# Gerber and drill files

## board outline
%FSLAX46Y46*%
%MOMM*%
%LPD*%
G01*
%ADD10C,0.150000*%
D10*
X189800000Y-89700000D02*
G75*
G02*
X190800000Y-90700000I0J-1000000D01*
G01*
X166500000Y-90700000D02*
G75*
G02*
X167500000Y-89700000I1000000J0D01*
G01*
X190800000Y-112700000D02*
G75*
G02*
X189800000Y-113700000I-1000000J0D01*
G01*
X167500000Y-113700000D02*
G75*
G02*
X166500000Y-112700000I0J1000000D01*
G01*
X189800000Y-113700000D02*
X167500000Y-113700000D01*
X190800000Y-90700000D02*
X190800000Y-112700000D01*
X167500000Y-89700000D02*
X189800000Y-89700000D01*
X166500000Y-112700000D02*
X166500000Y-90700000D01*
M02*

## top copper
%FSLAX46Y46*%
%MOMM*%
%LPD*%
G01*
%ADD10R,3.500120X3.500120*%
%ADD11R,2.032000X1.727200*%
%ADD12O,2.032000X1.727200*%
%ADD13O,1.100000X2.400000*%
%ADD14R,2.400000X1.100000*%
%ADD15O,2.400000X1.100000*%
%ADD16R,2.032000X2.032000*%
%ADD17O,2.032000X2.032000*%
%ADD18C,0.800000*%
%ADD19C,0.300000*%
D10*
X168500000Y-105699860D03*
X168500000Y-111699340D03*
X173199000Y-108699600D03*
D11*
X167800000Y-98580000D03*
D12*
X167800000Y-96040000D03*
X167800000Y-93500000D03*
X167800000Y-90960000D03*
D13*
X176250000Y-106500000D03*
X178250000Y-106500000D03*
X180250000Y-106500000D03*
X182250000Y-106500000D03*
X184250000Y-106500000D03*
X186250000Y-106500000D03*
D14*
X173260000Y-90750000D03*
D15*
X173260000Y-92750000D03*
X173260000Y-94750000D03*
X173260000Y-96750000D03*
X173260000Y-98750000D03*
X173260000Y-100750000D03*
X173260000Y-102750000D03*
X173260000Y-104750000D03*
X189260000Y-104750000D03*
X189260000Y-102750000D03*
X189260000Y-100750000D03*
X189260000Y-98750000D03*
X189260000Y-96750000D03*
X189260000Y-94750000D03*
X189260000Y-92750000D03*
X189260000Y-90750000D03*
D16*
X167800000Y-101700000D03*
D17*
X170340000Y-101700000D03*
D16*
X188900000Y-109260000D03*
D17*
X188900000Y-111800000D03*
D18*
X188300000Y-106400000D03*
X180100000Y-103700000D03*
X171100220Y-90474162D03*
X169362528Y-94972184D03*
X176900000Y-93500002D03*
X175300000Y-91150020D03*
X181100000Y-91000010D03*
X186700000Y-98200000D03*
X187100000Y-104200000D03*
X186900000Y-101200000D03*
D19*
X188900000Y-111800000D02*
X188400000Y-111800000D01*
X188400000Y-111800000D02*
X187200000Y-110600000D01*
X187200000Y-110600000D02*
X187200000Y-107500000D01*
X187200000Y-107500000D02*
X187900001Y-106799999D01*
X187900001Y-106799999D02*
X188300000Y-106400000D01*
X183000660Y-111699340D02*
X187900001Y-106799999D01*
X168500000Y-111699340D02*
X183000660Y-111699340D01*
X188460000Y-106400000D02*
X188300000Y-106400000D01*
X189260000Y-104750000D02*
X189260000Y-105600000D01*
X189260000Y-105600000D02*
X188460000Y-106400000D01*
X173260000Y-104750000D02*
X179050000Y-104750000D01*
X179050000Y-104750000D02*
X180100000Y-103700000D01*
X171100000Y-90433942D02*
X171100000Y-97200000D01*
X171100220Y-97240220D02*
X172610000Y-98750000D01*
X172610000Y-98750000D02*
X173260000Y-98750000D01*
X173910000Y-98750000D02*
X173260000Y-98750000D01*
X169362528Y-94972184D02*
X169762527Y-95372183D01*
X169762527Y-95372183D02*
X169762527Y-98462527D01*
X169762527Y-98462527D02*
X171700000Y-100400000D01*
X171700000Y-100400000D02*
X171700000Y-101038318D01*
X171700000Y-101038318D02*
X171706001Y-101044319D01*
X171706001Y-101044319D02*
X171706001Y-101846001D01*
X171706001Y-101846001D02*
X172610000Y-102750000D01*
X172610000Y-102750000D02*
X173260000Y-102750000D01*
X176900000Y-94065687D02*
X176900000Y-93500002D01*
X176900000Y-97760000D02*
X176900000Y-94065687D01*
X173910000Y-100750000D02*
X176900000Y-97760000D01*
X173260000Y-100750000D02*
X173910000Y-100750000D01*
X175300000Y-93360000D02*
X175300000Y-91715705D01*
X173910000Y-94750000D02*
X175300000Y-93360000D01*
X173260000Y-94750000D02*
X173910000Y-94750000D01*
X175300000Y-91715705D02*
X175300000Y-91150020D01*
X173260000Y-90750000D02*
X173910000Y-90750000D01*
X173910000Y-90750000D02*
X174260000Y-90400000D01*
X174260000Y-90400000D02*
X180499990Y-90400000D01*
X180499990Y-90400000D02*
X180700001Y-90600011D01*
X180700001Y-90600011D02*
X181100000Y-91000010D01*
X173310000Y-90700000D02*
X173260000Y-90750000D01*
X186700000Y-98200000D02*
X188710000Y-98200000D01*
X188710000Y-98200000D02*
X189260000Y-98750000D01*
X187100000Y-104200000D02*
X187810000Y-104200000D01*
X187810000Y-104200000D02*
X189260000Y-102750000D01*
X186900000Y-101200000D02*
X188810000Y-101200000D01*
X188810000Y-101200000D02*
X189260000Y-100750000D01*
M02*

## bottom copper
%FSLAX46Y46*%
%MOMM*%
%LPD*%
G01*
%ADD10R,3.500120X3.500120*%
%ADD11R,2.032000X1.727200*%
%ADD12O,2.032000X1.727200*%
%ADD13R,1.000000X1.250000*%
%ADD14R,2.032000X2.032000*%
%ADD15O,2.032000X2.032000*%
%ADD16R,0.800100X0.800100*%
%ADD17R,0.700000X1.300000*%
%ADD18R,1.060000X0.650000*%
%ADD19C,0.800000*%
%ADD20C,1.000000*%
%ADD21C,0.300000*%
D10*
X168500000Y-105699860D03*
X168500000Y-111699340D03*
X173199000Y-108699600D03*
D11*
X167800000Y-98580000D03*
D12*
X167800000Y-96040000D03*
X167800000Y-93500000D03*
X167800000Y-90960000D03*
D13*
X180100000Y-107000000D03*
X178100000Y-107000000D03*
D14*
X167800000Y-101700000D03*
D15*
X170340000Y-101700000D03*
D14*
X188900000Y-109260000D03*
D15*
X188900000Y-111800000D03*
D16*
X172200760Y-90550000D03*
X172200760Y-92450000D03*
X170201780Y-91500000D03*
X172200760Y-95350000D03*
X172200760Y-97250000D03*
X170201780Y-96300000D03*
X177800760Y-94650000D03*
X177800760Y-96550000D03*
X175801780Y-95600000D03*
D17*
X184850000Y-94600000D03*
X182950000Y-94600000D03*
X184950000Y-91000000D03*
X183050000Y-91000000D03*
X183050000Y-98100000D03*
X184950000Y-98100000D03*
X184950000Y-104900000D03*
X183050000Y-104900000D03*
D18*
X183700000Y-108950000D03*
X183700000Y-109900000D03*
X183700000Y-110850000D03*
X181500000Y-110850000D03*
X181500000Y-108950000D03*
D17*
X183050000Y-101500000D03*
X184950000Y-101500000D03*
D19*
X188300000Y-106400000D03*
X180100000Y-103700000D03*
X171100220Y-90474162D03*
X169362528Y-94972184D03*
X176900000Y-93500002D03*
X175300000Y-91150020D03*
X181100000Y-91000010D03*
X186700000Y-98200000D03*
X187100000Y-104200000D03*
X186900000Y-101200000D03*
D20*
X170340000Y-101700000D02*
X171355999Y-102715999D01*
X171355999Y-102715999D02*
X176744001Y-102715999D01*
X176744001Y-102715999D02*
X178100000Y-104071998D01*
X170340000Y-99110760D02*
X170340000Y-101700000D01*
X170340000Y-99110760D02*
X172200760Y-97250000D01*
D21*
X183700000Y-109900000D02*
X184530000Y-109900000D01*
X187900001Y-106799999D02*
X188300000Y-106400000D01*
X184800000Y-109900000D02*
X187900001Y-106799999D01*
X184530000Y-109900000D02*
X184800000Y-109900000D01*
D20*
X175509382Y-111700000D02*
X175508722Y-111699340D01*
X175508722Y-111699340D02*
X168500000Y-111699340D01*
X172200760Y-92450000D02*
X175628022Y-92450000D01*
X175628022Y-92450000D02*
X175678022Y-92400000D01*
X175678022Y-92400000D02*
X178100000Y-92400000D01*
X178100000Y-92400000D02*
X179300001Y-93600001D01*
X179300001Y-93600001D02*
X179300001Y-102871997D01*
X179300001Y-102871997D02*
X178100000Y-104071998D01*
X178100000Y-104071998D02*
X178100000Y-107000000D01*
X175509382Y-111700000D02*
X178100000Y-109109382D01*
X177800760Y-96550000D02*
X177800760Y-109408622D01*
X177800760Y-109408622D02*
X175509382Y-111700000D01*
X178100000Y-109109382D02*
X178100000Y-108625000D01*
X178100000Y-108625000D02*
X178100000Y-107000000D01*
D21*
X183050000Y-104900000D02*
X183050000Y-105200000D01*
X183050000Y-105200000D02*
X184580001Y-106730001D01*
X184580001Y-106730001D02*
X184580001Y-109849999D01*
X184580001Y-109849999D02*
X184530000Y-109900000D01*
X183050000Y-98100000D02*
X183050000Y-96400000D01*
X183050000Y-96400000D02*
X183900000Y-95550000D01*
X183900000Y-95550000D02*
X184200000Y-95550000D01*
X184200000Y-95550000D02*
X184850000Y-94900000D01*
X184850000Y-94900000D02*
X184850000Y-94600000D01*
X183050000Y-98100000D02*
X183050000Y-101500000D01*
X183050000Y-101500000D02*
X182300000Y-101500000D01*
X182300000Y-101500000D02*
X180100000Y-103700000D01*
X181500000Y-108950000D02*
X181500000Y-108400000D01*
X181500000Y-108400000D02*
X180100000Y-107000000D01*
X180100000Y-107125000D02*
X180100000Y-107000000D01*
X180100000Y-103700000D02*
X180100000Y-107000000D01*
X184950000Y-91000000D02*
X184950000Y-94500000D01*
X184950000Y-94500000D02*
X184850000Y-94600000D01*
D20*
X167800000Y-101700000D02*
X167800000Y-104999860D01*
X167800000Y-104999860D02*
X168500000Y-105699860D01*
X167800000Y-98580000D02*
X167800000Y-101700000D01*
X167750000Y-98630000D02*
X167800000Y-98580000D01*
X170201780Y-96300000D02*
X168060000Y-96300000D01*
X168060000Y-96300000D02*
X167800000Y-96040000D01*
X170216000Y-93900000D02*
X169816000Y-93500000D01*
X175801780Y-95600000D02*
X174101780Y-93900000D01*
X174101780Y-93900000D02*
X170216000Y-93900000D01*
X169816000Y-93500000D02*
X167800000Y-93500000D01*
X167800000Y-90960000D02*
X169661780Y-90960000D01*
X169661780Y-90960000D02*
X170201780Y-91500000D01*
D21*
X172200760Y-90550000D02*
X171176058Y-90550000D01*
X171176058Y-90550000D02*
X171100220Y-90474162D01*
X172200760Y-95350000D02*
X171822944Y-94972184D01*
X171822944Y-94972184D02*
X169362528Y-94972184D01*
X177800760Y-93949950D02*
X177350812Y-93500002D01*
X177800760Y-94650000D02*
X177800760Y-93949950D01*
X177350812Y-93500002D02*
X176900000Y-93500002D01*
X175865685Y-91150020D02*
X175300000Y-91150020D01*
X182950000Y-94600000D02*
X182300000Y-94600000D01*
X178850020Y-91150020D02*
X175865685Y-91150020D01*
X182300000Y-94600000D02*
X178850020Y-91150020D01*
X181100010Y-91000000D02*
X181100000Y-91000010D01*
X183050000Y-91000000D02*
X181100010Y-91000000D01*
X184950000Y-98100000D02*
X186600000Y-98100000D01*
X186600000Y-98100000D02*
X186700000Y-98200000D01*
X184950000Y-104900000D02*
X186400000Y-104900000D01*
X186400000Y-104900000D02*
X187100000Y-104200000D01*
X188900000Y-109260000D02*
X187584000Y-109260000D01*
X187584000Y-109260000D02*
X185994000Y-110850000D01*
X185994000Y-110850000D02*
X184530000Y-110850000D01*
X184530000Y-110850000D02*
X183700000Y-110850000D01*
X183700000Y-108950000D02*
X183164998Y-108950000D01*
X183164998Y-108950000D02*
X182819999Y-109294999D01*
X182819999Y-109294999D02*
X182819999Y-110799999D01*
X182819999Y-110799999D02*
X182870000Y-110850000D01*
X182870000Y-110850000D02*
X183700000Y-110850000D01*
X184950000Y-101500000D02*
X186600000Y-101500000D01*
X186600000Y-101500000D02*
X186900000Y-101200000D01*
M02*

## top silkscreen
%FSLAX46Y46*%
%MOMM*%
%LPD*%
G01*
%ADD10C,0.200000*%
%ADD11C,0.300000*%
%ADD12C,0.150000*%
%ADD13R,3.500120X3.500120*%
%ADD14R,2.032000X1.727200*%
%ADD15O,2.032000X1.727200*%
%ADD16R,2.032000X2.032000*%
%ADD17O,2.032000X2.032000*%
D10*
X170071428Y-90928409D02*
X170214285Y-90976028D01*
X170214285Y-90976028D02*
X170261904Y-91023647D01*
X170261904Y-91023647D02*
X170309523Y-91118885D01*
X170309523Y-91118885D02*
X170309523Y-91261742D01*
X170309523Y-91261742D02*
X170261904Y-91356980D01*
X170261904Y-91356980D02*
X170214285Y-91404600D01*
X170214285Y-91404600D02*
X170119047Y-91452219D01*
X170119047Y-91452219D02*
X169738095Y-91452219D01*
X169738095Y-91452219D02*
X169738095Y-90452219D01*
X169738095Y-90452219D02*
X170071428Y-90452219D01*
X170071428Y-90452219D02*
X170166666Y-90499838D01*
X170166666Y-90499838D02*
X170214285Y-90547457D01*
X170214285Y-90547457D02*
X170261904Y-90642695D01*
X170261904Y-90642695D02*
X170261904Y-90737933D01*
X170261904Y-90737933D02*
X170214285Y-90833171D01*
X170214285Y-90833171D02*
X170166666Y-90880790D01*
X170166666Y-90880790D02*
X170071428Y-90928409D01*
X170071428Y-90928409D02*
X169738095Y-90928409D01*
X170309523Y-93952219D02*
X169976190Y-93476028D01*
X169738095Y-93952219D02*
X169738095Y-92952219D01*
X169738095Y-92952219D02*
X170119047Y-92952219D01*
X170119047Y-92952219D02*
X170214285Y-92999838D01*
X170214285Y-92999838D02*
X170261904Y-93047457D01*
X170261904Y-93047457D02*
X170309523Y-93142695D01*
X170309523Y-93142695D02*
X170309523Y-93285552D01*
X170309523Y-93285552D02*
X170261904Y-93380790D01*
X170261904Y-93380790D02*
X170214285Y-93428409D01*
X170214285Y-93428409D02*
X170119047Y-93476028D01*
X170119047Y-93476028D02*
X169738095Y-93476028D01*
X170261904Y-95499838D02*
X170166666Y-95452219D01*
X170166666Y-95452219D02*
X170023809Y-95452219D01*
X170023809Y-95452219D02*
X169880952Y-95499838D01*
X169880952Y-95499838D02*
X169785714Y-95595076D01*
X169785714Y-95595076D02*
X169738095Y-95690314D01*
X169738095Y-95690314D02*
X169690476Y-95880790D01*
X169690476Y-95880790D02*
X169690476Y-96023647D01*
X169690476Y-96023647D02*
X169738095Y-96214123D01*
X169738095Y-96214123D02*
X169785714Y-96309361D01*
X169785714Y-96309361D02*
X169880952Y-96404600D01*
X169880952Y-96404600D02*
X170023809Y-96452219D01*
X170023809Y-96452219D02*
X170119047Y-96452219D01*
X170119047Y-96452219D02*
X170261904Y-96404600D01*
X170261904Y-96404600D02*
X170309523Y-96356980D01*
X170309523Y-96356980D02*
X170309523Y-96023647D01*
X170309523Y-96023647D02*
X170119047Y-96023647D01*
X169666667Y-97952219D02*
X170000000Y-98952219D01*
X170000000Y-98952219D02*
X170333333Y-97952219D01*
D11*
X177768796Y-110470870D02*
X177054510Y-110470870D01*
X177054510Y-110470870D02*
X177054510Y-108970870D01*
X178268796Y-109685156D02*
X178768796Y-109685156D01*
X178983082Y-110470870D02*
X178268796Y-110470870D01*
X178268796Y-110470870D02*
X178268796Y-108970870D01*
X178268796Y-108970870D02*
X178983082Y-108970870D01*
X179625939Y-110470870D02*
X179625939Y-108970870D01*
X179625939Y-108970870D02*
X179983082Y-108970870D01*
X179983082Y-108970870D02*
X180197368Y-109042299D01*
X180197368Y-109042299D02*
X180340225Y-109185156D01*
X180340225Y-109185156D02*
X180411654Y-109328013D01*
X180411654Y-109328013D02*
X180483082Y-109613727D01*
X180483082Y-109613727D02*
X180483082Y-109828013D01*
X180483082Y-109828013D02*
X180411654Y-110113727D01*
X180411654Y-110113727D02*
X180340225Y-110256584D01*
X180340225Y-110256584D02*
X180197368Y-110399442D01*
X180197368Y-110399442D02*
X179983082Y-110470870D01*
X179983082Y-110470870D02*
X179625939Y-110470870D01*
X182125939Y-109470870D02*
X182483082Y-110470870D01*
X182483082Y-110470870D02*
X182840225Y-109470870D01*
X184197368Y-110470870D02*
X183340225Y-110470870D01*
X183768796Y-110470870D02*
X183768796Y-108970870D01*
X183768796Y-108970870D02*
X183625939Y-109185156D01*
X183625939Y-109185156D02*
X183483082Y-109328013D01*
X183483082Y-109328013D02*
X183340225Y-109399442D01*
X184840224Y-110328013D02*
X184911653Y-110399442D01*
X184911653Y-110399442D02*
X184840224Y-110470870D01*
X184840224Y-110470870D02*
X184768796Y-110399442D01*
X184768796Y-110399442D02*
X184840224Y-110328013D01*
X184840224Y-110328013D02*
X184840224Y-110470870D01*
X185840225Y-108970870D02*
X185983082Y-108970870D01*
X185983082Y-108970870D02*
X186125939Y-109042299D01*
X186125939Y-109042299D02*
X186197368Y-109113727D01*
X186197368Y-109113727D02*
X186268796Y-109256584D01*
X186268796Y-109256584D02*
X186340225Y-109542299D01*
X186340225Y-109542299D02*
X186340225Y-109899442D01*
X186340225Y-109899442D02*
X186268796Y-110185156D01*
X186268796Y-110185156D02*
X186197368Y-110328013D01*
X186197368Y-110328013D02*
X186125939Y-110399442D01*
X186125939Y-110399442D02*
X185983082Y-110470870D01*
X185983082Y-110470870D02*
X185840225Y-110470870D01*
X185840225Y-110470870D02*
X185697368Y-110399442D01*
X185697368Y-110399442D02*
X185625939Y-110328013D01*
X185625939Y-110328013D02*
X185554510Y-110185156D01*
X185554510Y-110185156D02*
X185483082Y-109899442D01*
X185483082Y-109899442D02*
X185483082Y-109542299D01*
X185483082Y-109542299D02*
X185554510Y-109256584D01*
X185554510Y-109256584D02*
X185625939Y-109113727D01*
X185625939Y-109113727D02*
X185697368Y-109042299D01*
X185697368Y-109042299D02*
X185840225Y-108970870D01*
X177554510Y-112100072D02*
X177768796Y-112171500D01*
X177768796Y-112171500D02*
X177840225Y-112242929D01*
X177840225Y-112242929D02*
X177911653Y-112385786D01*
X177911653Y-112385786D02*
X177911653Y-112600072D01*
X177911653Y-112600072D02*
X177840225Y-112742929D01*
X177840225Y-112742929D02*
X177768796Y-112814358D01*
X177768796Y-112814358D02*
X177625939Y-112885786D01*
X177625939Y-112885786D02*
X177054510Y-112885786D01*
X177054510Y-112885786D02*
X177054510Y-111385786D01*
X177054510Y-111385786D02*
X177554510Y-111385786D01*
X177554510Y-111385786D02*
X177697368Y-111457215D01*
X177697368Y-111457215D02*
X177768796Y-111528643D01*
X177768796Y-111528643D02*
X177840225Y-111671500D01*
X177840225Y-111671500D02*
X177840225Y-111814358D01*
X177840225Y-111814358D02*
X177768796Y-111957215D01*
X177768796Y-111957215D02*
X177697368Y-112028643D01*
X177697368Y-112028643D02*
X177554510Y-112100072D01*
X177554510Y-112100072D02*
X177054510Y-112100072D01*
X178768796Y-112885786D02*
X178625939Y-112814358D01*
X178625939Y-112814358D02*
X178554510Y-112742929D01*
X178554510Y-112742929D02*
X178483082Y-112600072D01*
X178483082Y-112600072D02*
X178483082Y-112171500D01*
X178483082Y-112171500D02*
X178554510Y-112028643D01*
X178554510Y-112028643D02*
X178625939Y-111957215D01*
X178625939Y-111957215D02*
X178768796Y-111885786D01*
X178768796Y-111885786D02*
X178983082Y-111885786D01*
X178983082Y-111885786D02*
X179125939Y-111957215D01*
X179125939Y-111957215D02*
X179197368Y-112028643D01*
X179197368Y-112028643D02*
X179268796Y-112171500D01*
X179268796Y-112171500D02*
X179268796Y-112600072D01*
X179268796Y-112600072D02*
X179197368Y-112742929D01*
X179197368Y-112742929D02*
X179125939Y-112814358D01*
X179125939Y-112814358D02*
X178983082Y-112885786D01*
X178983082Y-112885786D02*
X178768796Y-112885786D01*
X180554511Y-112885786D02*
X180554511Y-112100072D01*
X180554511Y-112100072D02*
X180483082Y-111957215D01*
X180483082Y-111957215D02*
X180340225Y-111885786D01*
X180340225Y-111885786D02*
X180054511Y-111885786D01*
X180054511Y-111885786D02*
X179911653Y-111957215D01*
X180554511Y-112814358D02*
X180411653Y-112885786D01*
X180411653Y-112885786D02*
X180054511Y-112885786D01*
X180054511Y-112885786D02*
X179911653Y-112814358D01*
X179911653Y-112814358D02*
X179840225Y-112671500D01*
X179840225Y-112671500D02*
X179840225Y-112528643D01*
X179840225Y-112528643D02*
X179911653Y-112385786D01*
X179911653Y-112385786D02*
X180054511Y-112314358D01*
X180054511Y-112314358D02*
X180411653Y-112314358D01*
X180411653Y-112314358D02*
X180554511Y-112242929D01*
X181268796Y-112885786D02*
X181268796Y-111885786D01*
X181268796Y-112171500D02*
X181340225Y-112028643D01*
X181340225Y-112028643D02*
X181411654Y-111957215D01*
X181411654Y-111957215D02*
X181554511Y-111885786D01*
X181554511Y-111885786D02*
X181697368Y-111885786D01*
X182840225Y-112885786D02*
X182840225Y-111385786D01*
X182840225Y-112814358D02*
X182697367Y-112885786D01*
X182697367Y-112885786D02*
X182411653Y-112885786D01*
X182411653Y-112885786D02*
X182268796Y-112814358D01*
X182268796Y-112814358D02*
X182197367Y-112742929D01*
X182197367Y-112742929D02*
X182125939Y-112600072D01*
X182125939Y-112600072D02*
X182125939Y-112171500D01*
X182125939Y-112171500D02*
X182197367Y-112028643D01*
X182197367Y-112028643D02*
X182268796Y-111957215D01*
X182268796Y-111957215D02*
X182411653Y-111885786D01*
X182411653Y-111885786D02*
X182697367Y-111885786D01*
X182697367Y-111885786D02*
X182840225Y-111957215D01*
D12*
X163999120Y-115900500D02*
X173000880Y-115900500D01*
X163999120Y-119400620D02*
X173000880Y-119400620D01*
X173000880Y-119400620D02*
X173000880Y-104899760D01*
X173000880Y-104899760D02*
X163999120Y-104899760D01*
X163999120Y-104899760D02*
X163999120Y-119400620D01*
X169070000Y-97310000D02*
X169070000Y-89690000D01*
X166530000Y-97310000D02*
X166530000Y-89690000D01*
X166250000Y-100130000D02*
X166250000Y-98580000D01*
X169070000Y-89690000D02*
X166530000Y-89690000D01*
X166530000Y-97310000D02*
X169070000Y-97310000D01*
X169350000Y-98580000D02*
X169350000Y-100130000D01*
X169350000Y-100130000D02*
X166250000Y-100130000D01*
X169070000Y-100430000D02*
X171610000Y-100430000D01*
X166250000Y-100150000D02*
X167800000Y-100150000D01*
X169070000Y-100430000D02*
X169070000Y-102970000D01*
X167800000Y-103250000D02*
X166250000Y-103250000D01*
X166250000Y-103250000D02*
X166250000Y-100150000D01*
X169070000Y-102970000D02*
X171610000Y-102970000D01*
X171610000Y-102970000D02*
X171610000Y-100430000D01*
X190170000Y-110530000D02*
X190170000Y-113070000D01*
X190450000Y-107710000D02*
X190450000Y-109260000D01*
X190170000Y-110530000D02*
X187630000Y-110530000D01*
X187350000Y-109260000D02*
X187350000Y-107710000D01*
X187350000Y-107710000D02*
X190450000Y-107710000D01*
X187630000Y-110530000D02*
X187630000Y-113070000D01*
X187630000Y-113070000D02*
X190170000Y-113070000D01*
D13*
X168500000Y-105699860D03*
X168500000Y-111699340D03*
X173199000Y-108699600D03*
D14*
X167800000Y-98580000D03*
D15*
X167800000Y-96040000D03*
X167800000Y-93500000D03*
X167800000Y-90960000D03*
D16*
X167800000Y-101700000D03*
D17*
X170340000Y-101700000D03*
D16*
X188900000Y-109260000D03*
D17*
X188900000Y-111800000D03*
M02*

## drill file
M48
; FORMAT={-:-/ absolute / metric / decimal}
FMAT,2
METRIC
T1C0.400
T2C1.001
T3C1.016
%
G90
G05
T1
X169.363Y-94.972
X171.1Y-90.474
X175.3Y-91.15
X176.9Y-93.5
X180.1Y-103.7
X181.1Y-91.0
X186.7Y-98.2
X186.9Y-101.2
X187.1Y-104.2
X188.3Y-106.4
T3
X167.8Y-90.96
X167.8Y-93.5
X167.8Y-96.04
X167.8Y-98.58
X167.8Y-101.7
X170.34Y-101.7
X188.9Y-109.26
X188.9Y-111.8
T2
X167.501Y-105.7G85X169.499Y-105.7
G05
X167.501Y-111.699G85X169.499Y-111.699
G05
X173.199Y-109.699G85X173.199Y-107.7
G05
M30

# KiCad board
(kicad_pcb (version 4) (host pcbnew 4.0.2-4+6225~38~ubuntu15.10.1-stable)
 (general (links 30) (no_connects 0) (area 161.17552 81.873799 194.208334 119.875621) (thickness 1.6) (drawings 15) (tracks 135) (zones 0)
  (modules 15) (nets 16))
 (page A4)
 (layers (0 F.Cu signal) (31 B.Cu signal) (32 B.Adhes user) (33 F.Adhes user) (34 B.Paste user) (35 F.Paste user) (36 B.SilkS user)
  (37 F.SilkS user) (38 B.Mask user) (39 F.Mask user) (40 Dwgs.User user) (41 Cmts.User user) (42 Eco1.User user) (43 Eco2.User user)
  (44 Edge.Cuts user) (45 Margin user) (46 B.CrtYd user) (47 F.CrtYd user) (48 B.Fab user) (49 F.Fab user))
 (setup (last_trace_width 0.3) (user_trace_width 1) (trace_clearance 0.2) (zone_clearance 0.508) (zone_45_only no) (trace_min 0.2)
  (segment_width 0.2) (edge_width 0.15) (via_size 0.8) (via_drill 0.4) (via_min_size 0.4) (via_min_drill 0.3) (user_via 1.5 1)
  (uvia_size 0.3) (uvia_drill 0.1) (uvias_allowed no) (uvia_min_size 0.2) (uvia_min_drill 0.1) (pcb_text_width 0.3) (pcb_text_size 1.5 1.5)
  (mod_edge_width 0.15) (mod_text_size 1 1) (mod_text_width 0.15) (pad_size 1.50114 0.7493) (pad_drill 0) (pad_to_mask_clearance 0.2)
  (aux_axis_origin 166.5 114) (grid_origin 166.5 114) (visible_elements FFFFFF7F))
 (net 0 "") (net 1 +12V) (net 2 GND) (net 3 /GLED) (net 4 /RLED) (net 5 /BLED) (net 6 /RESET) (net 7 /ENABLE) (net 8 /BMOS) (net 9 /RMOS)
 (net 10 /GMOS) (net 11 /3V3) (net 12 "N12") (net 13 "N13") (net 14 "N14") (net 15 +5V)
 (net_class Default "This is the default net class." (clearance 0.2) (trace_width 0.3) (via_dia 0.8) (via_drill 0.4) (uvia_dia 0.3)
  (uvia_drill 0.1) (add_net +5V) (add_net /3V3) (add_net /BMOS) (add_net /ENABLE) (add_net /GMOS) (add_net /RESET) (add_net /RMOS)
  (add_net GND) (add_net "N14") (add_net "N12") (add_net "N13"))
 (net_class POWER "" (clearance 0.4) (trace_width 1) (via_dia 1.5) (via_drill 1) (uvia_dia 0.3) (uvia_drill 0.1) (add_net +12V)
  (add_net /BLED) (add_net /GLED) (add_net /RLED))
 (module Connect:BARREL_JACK (layer F.Cu) (at 168.5 111.9 90)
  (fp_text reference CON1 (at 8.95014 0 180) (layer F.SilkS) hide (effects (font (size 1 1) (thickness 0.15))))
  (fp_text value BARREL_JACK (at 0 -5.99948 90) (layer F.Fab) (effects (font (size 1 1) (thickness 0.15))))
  (fp_line (start -4.0005 -4.50088) (end -4.0005 4.50088) (layer F.SilkS) (width 0.15))
  (fp_line (start -7.50062 -4.50088) (end -7.50062 4.50088) (layer F.SilkS) (width 0.15))
  (fp_line (start -7.50062 4.50088) (end 7.00024 4.50088) (layer F.SilkS) (width 0.15))
  (fp_line (start 7.00024 4.50088) (end 7.00024 -4.50088) (layer F.SilkS) (width 0.15))
  (fp_line (start 7.00024 -4.50088) (end -7.50062 -4.50088) (layer F.SilkS) (width 0.15))
  (pad 1 thru_hole rect (at 6.20014 0 90) (size 3.50012 3.50012) (drill oval 1.00076 2.99974) (layers *.Cu *.Mask F.SilkS) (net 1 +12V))
  (pad 2 thru_hole rect (at 0.20066 0 90) (size 3.50012 3.50012) (drill oval 1.00076 2.99974) (layers *.Cu *.Mask F.SilkS) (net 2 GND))
  (pad 3 thru_hole rect (at 3.2004 4.699 90) (size 3.50012 3.50012) (drill oval 2.99974 1.00076) (layers *.Cu *.Mask F.SilkS)))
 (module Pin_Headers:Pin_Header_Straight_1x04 (layer F.Cu) (at 167.8 98.58 180)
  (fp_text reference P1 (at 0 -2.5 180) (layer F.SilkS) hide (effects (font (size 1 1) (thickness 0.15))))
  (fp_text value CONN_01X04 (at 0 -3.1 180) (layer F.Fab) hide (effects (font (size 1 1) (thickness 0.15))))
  (fp_line (start -1.27 1.27) (end -1.27 8.89) (layer F.SilkS) (width 0.15))
  (fp_line (start 1.27 1.27) (end 1.27 8.89) (layer F.SilkS) (width 0.15))
  (fp_line (start 1.55 -1.55) (end 1.55 0) (layer F.SilkS) (width 0.15))
  (fp_line (start -1.27 8.89) (end 1.27 8.89) (layer F.SilkS) (width 0.15))
  (fp_line (start 1.27 1.27) (end -1.27 1.27) (layer F.SilkS) (width 0.15))
  (fp_line (start -1.55 0) (end -1.55 -1.55) (layer F.SilkS) (width 0.15))
  (fp_line (start -1.55 -1.55) (end 1.55 -1.55) (layer F.SilkS) (width 0.15))
  (pad 1 thru_hole rect (at 0 0 180) (size 2.032 1.7272) (drill 1.016) (layers *.Cu *.Mask F.SilkS) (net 1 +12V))
  (pad 2 thru_hole oval (at 0 2.54 180) (size 2.032 1.7272) (drill 1.016) (layers *.Cu *.Mask F.SilkS) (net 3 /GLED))
  (pad 3 thru_hole oval (at 0 5.08 180) (size 2.032 1.7272) (drill 1.016) (layers *.Cu *.Mask F.SilkS) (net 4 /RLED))
  (pad 4 thru_hole oval (at 0 7.62 180) (size 2.032 1.7272) (drill 1.016) (layers *.Cu *.Mask F.SilkS) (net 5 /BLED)))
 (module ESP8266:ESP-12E (layer F.Cu) (at 173.26 90.75)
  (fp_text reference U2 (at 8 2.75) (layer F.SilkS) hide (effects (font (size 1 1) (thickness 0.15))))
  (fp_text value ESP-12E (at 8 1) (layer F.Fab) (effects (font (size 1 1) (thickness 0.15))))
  (pad 9 smd oval (at 2.99 15.75 90) (size 2.4 1.1) (layers F.Cu F.Paste F.Mask))
  (pad 10 smd oval (at 4.99 15.75 90) (size 2.4 1.1) (layers F.Cu F.Paste F.Mask))
  (pad 11 smd oval (at 6.99 15.75 90) (size 2.4 1.1) (layers F.Cu F.Paste F.Mask))
  (pad 12 smd oval (at 8.99 15.75 90) (size 2.4 1.1) (layers F.Cu F.Paste F.Mask))
  (pad 13 smd oval (at 10.99 15.75 90) (size 2.4 1.1) (layers F.Cu F.Paste F.Mask))
  (pad 14 smd oval (at 12.99 15.75 90) (size 2.4 1.1) (layers F.Cu F.Paste F.Mask))
  (pad 1 smd rect (at 0 0) (size 2.4 1.1) (layers F.Cu F.Paste F.Mask) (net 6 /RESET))
  (pad 2 smd oval (at 0 2) (size 2.4 1.1) (layers F.Cu F.Paste F.Mask))
  (pad 3 smd oval (at 0 4) (size 2.4 1.1) (layers F.Cu F.Paste F.Mask) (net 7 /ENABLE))
  (pad 4 smd oval (at 0 6) (size 2.4 1.1) (layers F.Cu F.Paste F.Mask))
  (pad 5 smd oval (at 0 8) (size 2.4 1.1) (layers F.Cu F.Paste F.Mask) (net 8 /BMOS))
  (pad 6 smd oval (at 0 10) (size 2.4 1.1) (layers F.Cu F.Paste F.Mask) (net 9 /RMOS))
  (pad 7 smd oval (at 0 12) (size 2.4 1.1) (layers F.Cu F.Paste F.Mask) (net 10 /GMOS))
  (pad 8 smd oval (at 0 14) (size 2.4 1.1) (layers F.Cu F.Paste F.Mask) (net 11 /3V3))
  (pad 15 smd oval (at 16 14) (size 2.4 1.1) (layers F.Cu F.Paste F.Mask) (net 2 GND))
  (pad 16 smd oval (at 16 12) (size 2.4 1.1) (layers F.Cu F.Paste F.Mask) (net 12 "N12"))
  (pad 17 smd oval (at 16 10) (size 2.4 1.1) (layers F.Cu F.Paste F.Mask) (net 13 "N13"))
  (pad 18 smd oval (at 16 8) (size 2.4 1.1) (layers F.Cu F.Paste F.Mask) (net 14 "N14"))
  (pad 19 smd oval (at 16 6) (size 2.4 1.1) (layers F.Cu F.Paste F.Mask))
  (pad 20 smd oval (at 16 4) (size 2.4 1.1) (layers F.Cu F.Paste F.Mask))
  (pad 21 smd oval (at 16 2) (size 2.4 1.1) (layers F.Cu F.Paste F.Mask))
  (pad 22 smd oval (at 16 0) (size 2.4 1.1) (layers F.Cu F.Paste F.Mask)))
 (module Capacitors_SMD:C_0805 (layer B.Cu) (at 179.1 107 180)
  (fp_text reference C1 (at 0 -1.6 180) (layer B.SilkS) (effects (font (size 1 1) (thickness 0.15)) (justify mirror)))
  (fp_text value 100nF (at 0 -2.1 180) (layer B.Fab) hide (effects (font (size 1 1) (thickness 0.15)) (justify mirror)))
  (pad 1 smd rect (at -1 0 180) (size 1 1.25) (layers B.Cu B.Paste B.Mask) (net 11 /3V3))
  (pad 2 smd rect (at 1 0 180) (size 1 1.25) (layers B.Cu B.Paste B.Mask) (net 2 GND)))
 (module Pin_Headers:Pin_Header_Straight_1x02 (layer F.Cu) (at 167.8 101.7 90)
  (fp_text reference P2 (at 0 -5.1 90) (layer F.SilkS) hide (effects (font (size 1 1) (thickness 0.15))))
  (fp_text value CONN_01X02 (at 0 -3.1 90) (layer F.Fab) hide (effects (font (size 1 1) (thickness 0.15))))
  (fp_line (start 1.27 1.27) (end 1.27 3.81) (layer F.SilkS) (width 0.15))
  (fp_line (start 1.55 -1.55) (end 1.55 0) (layer F.SilkS) (width 0.15))
  (fp_line (start 1.27 1.27) (end -1.27 1.27) (layer F.SilkS) (width 0.15))
  (fp_line (start -1.55 0) (end -1.55 -1.55) (layer F.SilkS) (width 0.15))
  (fp_line (start -1.55 -1.55) (end 1.55 -1.55) (layer F.SilkS) (width 0.15))
  (fp_line (start -1.27 1.27) (end -1.27 3.81) (layer F.SilkS) (width 0.15))
  (fp_line (start -1.27 3.81) (end 1.27 3.81) (layer F.SilkS) (width 0.15))
  (pad 1 thru_hole rect (at 0 0 90) (size 2.032 2.032) (drill 1.016) (layers *.Cu *.Mask F.SilkS) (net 1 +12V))
  (pad 2 thru_hole oval (at 0 2.54 90) (size 2.032 2.032) (drill 1.016) (layers *.Cu *.Mask F.SilkS) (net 2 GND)))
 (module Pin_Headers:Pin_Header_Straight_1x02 (layer F.Cu) (at 188.9 109.26)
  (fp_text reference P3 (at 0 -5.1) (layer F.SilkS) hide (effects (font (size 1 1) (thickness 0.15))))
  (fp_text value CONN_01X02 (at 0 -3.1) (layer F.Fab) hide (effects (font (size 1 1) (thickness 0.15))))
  (fp_line (start 1.27 1.27) (end 1.27 3.81) (layer F.SilkS) (width 0.15))
  (fp_line (start 1.55 -1.55) (end 1.55 0) (layer F.SilkS) (width 0.15))
  (fp_line (start 1.27 1.27) (end -1.27 1.27) (layer F.SilkS) (width 0.15))
  (fp_line (start -1.55 0) (end -1.55 -1.55) (layer F.SilkS) (width 0.15))
  (fp_line (start -1.55 -1.55) (end 1.55 -1.55) (layer F.SilkS) (width 0.15))
  (fp_line (start -1.27 1.27) (end -1.27 3.81) (layer F.SilkS) (width 0.15))
  (fp_line (start -1.27 3.81) (end 1.27 3.81) (layer F.SilkS) (width 0.15))
  (pad 1 thru_hole rect (at 0 0) (size 2.032 2.032) (drill 1.016) (layers *.Cu *.Mask F.SilkS) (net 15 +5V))
  (pad 2 thru_hole oval (at 0 2.54) (size 2.032 2.032) (drill 1.016) (layers *.Cu *.Mask F.SilkS) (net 2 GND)))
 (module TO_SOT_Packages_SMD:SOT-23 (layer B.Cu) (at 171.2 91.5 270)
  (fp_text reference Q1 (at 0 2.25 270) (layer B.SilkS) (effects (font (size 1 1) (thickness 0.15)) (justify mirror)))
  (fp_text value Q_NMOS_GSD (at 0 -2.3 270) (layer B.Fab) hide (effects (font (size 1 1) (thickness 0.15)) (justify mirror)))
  (pad 1 smd rect (at -0.95 -1.00076 270) (size 0.8001 0.8001) (layers B.Cu B.Paste B.Mask) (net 8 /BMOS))
  (pad 2 smd rect (at 0.95 -1.00076 270) (size 0.8001 0.8001) (layers B.Cu B.Paste B.Mask) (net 2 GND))
  (pad 3 smd rect (at 0 0.99822 270) (size 0.8001 0.8001) (layers B.Cu B.Paste B.Mask) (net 5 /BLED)))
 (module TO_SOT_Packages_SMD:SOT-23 (layer B.Cu) (at 171.2 96.3 270)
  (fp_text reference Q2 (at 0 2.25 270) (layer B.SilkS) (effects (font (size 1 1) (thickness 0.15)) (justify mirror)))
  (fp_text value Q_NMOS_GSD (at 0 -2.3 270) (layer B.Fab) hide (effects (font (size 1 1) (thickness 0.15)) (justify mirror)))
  (pad 1 smd rect (at -0.95 -1.00076 270) (size 0.8001 0.8001) (layers B.Cu B.Paste B.Mask) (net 10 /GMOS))
  (pad 2 smd rect (at 0.95 -1.00076 270) (size 0.8001 0.8001) (layers B.Cu B.Paste B.Mask) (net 2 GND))
  (pad 3 smd rect (at 0 0.99822 270) (size 0.8001 0.8001) (layers B.Cu B.Paste B.Mask) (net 3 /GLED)))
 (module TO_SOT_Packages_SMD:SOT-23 (layer B.Cu) (at 176.8 95.6 270)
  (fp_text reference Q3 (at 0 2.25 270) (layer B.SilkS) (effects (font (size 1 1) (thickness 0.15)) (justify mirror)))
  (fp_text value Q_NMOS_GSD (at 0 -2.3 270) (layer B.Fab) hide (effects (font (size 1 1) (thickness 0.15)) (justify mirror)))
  (pad 1 smd rect (at -0.95 -1.00076 270) (size 0.8001 0.8001) (layers B.Cu B.Paste B.Mask) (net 9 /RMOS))
  (pad 2 smd rect (at 0.95 -1.00076 270) (size 0.8001 0.8001) (layers B.Cu B.Paste B.Mask) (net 2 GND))
  (pad 3 smd rect (at 0 0.99822 270) (size 0.8001 0.8001) (layers B.Cu B.Paste B.Mask) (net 4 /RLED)))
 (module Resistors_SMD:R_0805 (layer B.Cu) (at 183.9 94.6 180)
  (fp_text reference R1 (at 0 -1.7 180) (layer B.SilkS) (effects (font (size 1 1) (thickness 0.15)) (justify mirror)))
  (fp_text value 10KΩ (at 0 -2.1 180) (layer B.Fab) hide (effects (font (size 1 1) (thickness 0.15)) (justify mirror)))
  (pad 1 smd rect (at -0.95 0 180) (size 0.7 1.3) (layers B.Cu B.Paste B.Mask) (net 11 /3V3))
  (pad 2 smd rect (at 0.95 0 180) (size 0.7 1.3) (layers B.Cu B.Paste B.Mask) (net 7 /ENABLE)))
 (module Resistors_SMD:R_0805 (layer B.Cu) (at 184 91 180)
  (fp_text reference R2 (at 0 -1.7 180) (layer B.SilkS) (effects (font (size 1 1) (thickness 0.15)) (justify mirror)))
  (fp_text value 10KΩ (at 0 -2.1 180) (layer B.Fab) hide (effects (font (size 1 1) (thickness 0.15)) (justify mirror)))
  (pad 1 smd rect (at -0.95 0 180) (size 0.7 1.3) (layers B.Cu B.Paste B.Mask) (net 11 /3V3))
  (pad 2 smd rect (at 0.95 0 180) (size 0.7 1.3) (layers B.Cu B.Paste B.Mask) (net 6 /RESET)))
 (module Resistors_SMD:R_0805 (layer B.Cu) (at 184 98.1)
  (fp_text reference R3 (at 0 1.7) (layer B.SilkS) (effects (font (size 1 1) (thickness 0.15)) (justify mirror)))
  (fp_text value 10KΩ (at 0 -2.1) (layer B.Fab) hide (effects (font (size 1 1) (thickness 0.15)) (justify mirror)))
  (pad 1 smd rect (at -0.95 0) (size 0.7 1.3) (layers B.Cu B.Paste B.Mask) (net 11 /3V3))
  (pad 2 smd rect (at 0.95 0) (size 0.7 1.3) (layers B.Cu B.Paste B.Mask) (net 14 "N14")))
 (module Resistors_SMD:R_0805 (layer B.Cu) (at 184 104.9 180)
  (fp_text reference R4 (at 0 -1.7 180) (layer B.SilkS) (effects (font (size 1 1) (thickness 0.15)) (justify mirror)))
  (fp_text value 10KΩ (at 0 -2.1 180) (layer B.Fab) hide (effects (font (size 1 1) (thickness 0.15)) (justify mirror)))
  (pad 1 smd rect (at -0.95 0 180) (size 0.7 1.3) (layers B.Cu B.Paste B.Mask) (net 12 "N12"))
  (pad 2 smd rect (at 0.95 0 180) (size 0.7 1.3) (layers B.Cu B.Paste B.Mask) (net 2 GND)))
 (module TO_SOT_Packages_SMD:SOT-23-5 (layer B.Cu) (at 182.6 109.9 180)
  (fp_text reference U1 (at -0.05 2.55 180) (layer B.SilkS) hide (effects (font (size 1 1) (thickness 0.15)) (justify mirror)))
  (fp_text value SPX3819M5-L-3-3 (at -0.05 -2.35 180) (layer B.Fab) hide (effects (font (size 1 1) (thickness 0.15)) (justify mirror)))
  (pad 1 smd rect (at -1.1 0.95 180) (size 1.06 0.65) (layers B.Cu B.Paste B.Mask) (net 15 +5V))
  (pad 2 smd rect (at -1.1 0 180) (size 1.06 0.65) (layers B.Cu B.Paste B.Mask) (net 2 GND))
  (pad 3 smd rect (at -1.1 -0.95 180) (size 1.06 0.65) (layers B.Cu B.Paste B.Mask) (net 15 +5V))
  (pad 4 smd rect (at 1.1 -0.95 180) (size 1.06 0.65) (layers B.Cu B.Paste B.Mask))
  (pad 5 smd rect (at 1.1 0.95 180) (size 1.06 0.65) (layers B.Cu B.Paste B.Mask) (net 11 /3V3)))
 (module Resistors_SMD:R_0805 (layer B.Cu) (at 184 101.5)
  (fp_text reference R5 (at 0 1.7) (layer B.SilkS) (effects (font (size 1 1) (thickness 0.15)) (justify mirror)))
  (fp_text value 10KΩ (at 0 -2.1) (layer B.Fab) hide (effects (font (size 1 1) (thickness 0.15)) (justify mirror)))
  (pad 1 smd rect (at -0.95 0) (size 0.7 1.3) (layers B.Cu B.Paste B.Mask) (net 11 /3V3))
  (pad 2 smd rect (at 0.95 0) (size 0.7 1.3) (layers B.Cu B.Paste B.Mask) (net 13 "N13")))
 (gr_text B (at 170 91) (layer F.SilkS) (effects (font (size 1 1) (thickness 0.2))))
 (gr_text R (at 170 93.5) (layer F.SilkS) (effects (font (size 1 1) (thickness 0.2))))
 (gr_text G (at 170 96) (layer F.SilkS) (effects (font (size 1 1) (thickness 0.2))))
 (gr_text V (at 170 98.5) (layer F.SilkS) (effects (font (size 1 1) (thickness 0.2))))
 (gr_arc (start 189.8 90.7) (end 189.8 89.7) (angle 90) (layer Edge.Cuts) (width 0.15))
 (gr_arc (start 167.5 90.7) (end 166.5 90.7) (angle 90) (layer Edge.Cuts) (width 0.15))
 (gr_arc (start 189.8 112.7) (end 190.8 112.7) (angle 90) (layer Edge.Cuts) (width 0.15))
 (gr_arc (start 167.5 112.7) (end 167.5 113.7) (angle 90) (layer Edge.Cuts) (width 0.15))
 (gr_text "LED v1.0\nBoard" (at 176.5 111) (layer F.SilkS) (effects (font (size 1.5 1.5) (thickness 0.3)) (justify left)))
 (gr_line (start 189.8 113.7) (end 167.5 113.7) (layer Edge.Cuts) (width 0.15))
 (gr_line (start 190.8 90.7) (end 190.8 112.7) (layer Edge.Cuts) (width 0.15))
 (gr_line (start 167.5 89.7) (end 189.8 89.7) (layer Edge.Cuts) (width 0.15))
 (gr_line (start 166.5 112.7) (end 166.5 90.7) (layer Edge.Cuts) (width 0.15))
 (segment (start 170.34 101.7) (end 171.355999 102.715999) (width 1) (layer B.Cu) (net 2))
 (segment (start 171.355999 102.715999) (end 176.744001 102.715999) (width 1) (layer B.Cu) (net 2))
 (segment (start 176.744001 102.715999) (end 178.1 104.071998) (width 1) (layer B.Cu) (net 2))
 (segment (start 170.34 99.11076) (end 170.34 101.7) (width 1) (layer B.Cu) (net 2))
 (segment (start 170.34 99.11076) (end 172.20076 97.25) (width 1) (layer B.Cu) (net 2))
 (segment (start 188.9 111.8) (end 188.4 111.8) (width 0.3) (layer F.Cu) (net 2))
 (segment (start 188.4 111.8) (end 187.2 110.6) (width 0.3) (layer F.Cu) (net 2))
 (segment (start 187.2 110.6) (end 187.2 107.5) (width 0.3) (layer F.Cu) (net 2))
 (segment (start 187.2 107.5) (end 187.900001 106.799999) (width 0.3) (layer F.Cu) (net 2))
 (segment (start 187.900001 106.799999) (end 188.3 106.4) (width 0.3) (layer F.Cu) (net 2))
 (segment (start 183.7 109.9) (end 184.53 109.9) (width 0.3) (layer B.Cu) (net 2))
 (segment (start 183.00066 111.69934) (end 187.900001 106.799999) (width 0.3) (layer F.Cu) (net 2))
 (segment (start 168.5 111.69934) (end 183.00066 111.69934) (width 0.3) (layer F.Cu) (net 2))
 (segment (start 187.900001 106.799999) (end 188.3 106.4) (width 0.3) (layer B.Cu) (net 2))
 (segment (start 184.8 109.9) (end 187.900001 106.799999) (width 0.3) (layer B.Cu) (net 2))
 (segment (start 188.46 106.4) (end 188.3 106.4) (width 0.3) (layer F.Cu) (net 2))
 (segment (start 189.26 104.75) (end 189.26 105.6) (width 0.3) (layer F.Cu) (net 2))
 (segment (start 189.26 105.6) (end 188.46 106.4) (width 0.3) (layer F.Cu) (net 2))
 (via (at 188.3 106.4) (size 0.8) (drill 0.4) (layers F.Cu B.Cu) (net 2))
 (segment (start 184.53 109.9) (end 184.8 109.9) (width 0.3) (layer B.Cu) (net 2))
 (segment (start 175.509382 111.7) (end 175.508722 111.69934) (width 1) (layer B.Cu) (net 2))
 (segment (start 175.508722 111.69934) (end 168.5 111.69934) (width 1) (layer B.Cu) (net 2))
 (segment (start 172.20076 92.45) (end 175.628022 92.45) (width 1) (layer B.Cu) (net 2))
 (segment (start 175.628022 92.45) (end 175.678022 92.4) (width 1) (layer B.Cu) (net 2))
 (segment (start 175.678022 92.4) (end 178.1 92.4) (width 1) (layer B.Cu) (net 2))
 (segment (start 178.1 92.4) (end 179.300001 93.600001) (width 1) (layer B.Cu) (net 2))
 (segment (start 179.300001 93.600001) (end 179.300001 102.871997) (width 1) (layer B.Cu) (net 2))
 (segment (start 179.300001 102.871997) (end 178.1 104.071998) (width 1) (layer B.Cu) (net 2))
 (segment (start 178.1 104.071998) (end 178.1 107) (width 1) (layer B.Cu) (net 2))
 (segment (start 175.509382 111.7) (end 178.1 109.109382) (width 1) (layer B.Cu) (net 2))
 (segment (start 177.80076 96.55) (end 177.80076 109.408622) (width 1) (layer B.Cu) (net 2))
 (segment (start 177.80076 109.408622) (end 175.509382 111.7) (width 1) (layer B.Cu) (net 2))
 (segment (start 178.1 109.109382) (end 178.1 108.625) (width 1) (layer B.Cu) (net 2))
 (segment (start 178.1 108.625) (end 178.1 107) (width 1) (layer B.Cu) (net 2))
 (segment (start 183.05 104.9) (end 183.05 105.2) (width 0.3) (layer B.Cu) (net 2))
 (segment (start 183.05 105.2) (end 184.580001 106.730001) (width 0.3) (layer B.Cu) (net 2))
 (segment (start 184.580001 106.730001) (end 184.580001 109.849999) (width 0.3) (layer B.Cu) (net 2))
 (segment (start 184.580001 109.849999) (end 184.53 109.9) (width 0.3) (layer B.Cu) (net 2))
 (segment (start 183.05 98.1) (end 183.05 96.4) (width 0.3) (layer B.Cu) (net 11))
 (segment (start 183.05 96.4) (end 183.9 95.55) (width 0.3) (layer B.Cu) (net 11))
 (segment (start 183.9 95.55) (end 184.2 95.55) (width 0.3) (layer B.Cu) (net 11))
 (segment (start 184.2 95.55) (end 184.85 94.9) (width 0.3) (layer B.Cu) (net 11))
 (segment (start 184.85 94.9) (end 184.85 94.6) (width 0.3) (layer B.Cu) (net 11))
 (segment (start 183.05 98.1) (end 183.05 101.5) (width 0.3) (layer B.Cu) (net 11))
 (segment (start 183.05 101.5) (end 182.3 101.5) (width 0.3) (layer B.Cu) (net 11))
 (segment (start 182.3 101.5) (end 180.1 103.7) (width 0.3) (layer B.Cu) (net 11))
 (segment (start 181.5 108.95) (end 181.5 108.4) (width 0.3) (layer B.Cu) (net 11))
 (segment (start 181.5 108.4) (end 180.1 107) (width 0.3) (layer B.Cu) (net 11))
 (segment (start 180.1 107.125) (end 180.1 107) (width 0.3) (layer B.Cu) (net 11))
 (segment (start 173.26 104.75) (end 179.05 104.75) (width 0.3) (layer F.Cu) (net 11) (status 10))
 (segment (start 179.05 104.75) (end 180.1 103.7) (width 0.3) (layer F.Cu) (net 11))
 (via (at 180.1 103.7) (size 0.8) (drill 0.4) (layers F.Cu B.Cu) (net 11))
 (segment (start 180.1 103.7) (end 180.1 107) (width 0.3) (layer B.Cu) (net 11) (status 20))
 (segment (start 184.95 91) (end 184.95 94.5) (width 0.3) (layer B.Cu) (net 11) (status 30))
 (segment (start 184.95 94.5) (end 184.85 94.6) (width 0.3) (layer B.Cu) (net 11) (status 30))
 (segment (start 167.8 101.7) (end 167.8 104.99986) (width 1) (layer B.Cu) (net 1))
 (segment (start 167.8 104.99986) (end 168.5 105.69986) (width 1) (layer B.Cu) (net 1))
 (segment (start 167.8 98.58) (end 167.8 101.7) (width 1) (layer B.Cu) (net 1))
 (segment (start 167.75 98.63) (end 167.8 98.58) (width 1) (layer B.Cu) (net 1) (status 30))
 (segment (start 170.20178 96.3) (end 168.06 96.3) (width 1) (layer B.Cu) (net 3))
 (segment (start 168.06 96.3) (end 167.8 96.04) (width 1) (layer B.Cu) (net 3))
 (segment (start 170.216 93.9) (end 169.816 93.5) (width 1) (layer B.Cu) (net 4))
 (segment (start 175.80178 95.6) (end 174.10178 93.9) (width 1) (layer B.Cu) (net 4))
 (segment (start 174.10178 93.9) (end 170.216 93.9) (width 1) (layer B.Cu) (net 4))
 (segment (start 169.816 93.5) (end 167.8 93.5) (width 1) (layer B.Cu) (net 4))
 (segment (start 167.8 90.96) (end 169.66178 90.96) (width 1) (layer B.Cu) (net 5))
 (segment (start 169.66178 90.96) (end 170.20178 91.5) (width 1) (layer B.Cu) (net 5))
 (segment (start 171.1 90.433942) (end 171.1 97.2) (width 0.3) (layer F.Cu) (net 8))
 (segment (start 171.10022 97.24022) (end 172.61 98.75) (width 0.3) (layer F.Cu) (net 8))
 (segment (start 172.61 98.75) (end 173.26 98.75) (width 0.3) (layer F.Cu) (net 8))
 (segment (start 172.20076 90.55) (end 171.176058 90.55) (width 0.3) (layer B.Cu) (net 8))
 (via (at 171.10022 90.474162) (size 0.8) (drill 0.4) (layers F.Cu B.Cu) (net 8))
 (segment (start 171.176058 90.55) (end 171.10022 90.474162) (width 0.3) (layer B.Cu) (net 8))
 (segment (start 173.91 98.75) (end 173.26 98.75) (width 0.3) (layer F.Cu) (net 8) (status 30))
 (segment (start 169.362528 94.972184) (end 169.762527 95.372183) (width 0.3) (layer F.Cu) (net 10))
 (segment (start 169.762527 95.372183) (end 169.762527 98.462527) (width 0.3) (layer F.Cu) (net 10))
 (segment (start 169.762527 98.462527) (end 171.7 100.4) (width 0.3) (layer F.Cu) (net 10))
 (segment (start 171.7 100.4) (end 171.7 101.038318) (width 0.3) (layer F.Cu) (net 10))
 (segment (start 171.7 101.038318) (end 171.706001 101.044319) (width 0.3) (layer F.Cu) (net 10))
 (segment (start 171.706001 101.044319) (end 171.706001 101.846001) (width 0.3) (layer F.Cu) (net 10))
 (segment (start 171.706001 101.846001) (end 172.61 102.75) (width 0.3) (layer F.Cu) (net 10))
 (segment (start 172.61 102.75) (end 173.26 102.75) (width 0.3) (layer F.Cu) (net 10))
 (segment (start 172.20076 95.35) (end 171.822944 94.972184) (width 0.3) (layer B.Cu) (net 10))
 (segment (start 171.822944 94.972184) (end 169.362528 94.972184) (width 0.3) (layer B.Cu) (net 10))
 (via (at 169.362528 94.972184) (size 0.8) (drill 0.4) (layers F.Cu B.Cu) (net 10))
 (segment (start 177.80076 93.94995) (end 177.350812 93.500002) (width 0.3) (layer B.Cu) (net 9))
 (segment (start 176.9 94.065687) (end 176.9 93.500002) (width 0.3) (layer F.Cu) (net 9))
 (segment (start 176.9 97.76) (end 176.9 94.065687) (width 0.3) (layer F.Cu) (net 9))
 (segment (start 173.91 100.75) (end 176.9 97.76) (width 0.3) (layer F.Cu) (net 9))
 (via (at 176.9 93.500002) (size 0.8) (drill 0.4) (layers F.Cu B.Cu) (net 9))
 (segment (start 177.80076 94.65) (end 177.80076 93.94995) (width 0.3) (layer B.Cu) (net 9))
 (segment (start 173.26 100.75) (end 173.91 100.75) (width 0.3) (layer F.Cu) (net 9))
 (segment (start 177.350812 93.500002) (end 176.9 93.500002) (width 0.3) (layer B.Cu) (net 9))
 (segment (start 175.3 93.36) (end 175.3 91.715705) (width 0.3) (layer F.Cu) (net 7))
 (segment (start 173.91 94.75) (end 175.3 93.36) (width 0.3) (layer F.Cu) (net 7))
 (segment (start 173.26 94.75) (end 173.91 94.75) (width 0.3) (layer F.Cu) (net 7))
 (via (at 175.3 91.15002) (size 0.8) (drill 0.4) (layers F.Cu B.Cu) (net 7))
 (segment (start 175.865685 91.15002) (end 175.3 91.15002) (width 0.3) (layer B.Cu) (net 7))
 (segment (start 182.95 94.6) (end 182.3 94.6) (width 0.3) (layer B.Cu) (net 7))
 (segment (start 178.85002 91.15002) (end 175.865685 91.15002) (width 0.3) (layer B.Cu) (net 7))
 (segment (start 175.3 91.715705) (end 175.3 91.15002) (width 0.3) (layer F.Cu) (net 7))
 (segment (start 182.3 94.6) (end 178.85002 91.15002) (width 0.3) (layer B.Cu) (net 7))
 (segment (start 173.26 90.75) (end 173.91 90.75) (width 0.3) (layer F.Cu) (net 6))
 (segment (start 173.91 90.75) (end 174.26 90.4) (width 0.3) (layer F.Cu) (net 6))
 (segment (start 174.26 90.4) (end 180.49999 90.4) (width 0.3) (layer F.Cu) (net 6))
 (segment (start 180.49999 90.4) (end 180.700001 90.600011) (width 0.3) (layer F.Cu) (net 6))
 (segment (start 180.700001 90.600011) (end 181.1 91.00001) (width 0.3) (layer F.Cu) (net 6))
 (segment (start 181.10001 91) (end 181.1 91.00001) (width 0.3) (layer B.Cu) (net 6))
 (segment (start 183.05 91) (end 181.10001 91) (width 0.3) (layer B.Cu) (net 6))
 (via (at 181.1 91.00001) (size 0.8) (drill 0.4) (layers F.Cu B.Cu) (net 6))
 (segment (start 173.31 90.7) (end 173.26 90.75) (width 0.3) (layer F.Cu) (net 6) (status 30))
 (segment (start 186.7 98.2) (end 188.71 98.2) (width 0.3) (layer F.Cu) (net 14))
 (segment (start 188.71 98.2) (end 189.26 98.75) (width 0.3) (layer F.Cu) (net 14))
 (segment (start 184.95 98.1) (end 186.6 98.1) (width 0.3) (layer B.Cu) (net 14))
 (segment (start 186.6 98.1) (end 186.7 98.2) (width 0.3) (layer B.Cu) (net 14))
 (via (at 186.7 98.2) (size 0.8) (drill 0.4) (layers F.Cu B.Cu) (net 14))
 (segment (start 187.1 104.2) (end 187.81 104.2) (width 0.3) (layer F.Cu) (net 12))
 (segment (start 187.81 104.2) (end 189.26 102.75) (width 0.3) (layer F.Cu) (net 12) (status 20))
 (segment (start 184.95 104.9) (end 186.4 104.9) (width 0.3) (layer B.Cu) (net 12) (status 10))
 (segment (start 186.4 104.9) (end 187.1 104.2) (width 0.3) (layer B.Cu) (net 12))
 (via (at 187.1 104.2) (size 0.8) (drill 0.4) (layers F.Cu B.Cu) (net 12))
 (segment (start 188.9 109.26) (end 187.584 109.26) (width 0.3) (layer B.Cu) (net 15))
 (segment (start 187.584 109.26) (end 185.994 110.85) (width 0.3) (layer B.Cu) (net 15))
 (segment (start 185.994 110.85) (end 184.53 110.85) (width 0.3) (layer B.Cu) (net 15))
 (segment (start 184.53 110.85) (end 183.7 110.85) (width 0.3) (layer B.Cu) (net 15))
 (segment (start 183.7 108.95) (end 183.164998 108.95) (width 0.3) (layer B.Cu) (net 15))
 (segment (start 183.164998 108.95) (end 182.819999 109.294999) (width 0.3) (layer B.Cu) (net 15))
 (segment (start 182.819999 109.294999) (end 182.819999 110.799999) (width 0.3) (layer B.Cu) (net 15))
 (segment (start 182.819999 110.799999) (end 182.87 110.85) (width 0.3) (layer B.Cu) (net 15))
 (segment (start 182.87 110.85) (end 183.7 110.85) (width 0.3) (layer B.Cu) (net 15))
 (segment (start 186.9 101.2) (end 188.81 101.2) (width 0.3) (layer F.Cu) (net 13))
 (segment (start 188.81 101.2) (end 189.26 100.75) (width 0.3) (layer F.Cu) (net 13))
 (segment (start 184.95 101.5) (end 186.6 101.5) (width 0.3) (layer B.Cu) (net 13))
 (segment (start 186.6 101.5) (end 186.9 101.2) (width 0.3) (layer B.Cu) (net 13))
 (via (at 186.9 101.2) (size 0.8) (drill 0.4) (layers F.Cu B.Cu) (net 13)))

